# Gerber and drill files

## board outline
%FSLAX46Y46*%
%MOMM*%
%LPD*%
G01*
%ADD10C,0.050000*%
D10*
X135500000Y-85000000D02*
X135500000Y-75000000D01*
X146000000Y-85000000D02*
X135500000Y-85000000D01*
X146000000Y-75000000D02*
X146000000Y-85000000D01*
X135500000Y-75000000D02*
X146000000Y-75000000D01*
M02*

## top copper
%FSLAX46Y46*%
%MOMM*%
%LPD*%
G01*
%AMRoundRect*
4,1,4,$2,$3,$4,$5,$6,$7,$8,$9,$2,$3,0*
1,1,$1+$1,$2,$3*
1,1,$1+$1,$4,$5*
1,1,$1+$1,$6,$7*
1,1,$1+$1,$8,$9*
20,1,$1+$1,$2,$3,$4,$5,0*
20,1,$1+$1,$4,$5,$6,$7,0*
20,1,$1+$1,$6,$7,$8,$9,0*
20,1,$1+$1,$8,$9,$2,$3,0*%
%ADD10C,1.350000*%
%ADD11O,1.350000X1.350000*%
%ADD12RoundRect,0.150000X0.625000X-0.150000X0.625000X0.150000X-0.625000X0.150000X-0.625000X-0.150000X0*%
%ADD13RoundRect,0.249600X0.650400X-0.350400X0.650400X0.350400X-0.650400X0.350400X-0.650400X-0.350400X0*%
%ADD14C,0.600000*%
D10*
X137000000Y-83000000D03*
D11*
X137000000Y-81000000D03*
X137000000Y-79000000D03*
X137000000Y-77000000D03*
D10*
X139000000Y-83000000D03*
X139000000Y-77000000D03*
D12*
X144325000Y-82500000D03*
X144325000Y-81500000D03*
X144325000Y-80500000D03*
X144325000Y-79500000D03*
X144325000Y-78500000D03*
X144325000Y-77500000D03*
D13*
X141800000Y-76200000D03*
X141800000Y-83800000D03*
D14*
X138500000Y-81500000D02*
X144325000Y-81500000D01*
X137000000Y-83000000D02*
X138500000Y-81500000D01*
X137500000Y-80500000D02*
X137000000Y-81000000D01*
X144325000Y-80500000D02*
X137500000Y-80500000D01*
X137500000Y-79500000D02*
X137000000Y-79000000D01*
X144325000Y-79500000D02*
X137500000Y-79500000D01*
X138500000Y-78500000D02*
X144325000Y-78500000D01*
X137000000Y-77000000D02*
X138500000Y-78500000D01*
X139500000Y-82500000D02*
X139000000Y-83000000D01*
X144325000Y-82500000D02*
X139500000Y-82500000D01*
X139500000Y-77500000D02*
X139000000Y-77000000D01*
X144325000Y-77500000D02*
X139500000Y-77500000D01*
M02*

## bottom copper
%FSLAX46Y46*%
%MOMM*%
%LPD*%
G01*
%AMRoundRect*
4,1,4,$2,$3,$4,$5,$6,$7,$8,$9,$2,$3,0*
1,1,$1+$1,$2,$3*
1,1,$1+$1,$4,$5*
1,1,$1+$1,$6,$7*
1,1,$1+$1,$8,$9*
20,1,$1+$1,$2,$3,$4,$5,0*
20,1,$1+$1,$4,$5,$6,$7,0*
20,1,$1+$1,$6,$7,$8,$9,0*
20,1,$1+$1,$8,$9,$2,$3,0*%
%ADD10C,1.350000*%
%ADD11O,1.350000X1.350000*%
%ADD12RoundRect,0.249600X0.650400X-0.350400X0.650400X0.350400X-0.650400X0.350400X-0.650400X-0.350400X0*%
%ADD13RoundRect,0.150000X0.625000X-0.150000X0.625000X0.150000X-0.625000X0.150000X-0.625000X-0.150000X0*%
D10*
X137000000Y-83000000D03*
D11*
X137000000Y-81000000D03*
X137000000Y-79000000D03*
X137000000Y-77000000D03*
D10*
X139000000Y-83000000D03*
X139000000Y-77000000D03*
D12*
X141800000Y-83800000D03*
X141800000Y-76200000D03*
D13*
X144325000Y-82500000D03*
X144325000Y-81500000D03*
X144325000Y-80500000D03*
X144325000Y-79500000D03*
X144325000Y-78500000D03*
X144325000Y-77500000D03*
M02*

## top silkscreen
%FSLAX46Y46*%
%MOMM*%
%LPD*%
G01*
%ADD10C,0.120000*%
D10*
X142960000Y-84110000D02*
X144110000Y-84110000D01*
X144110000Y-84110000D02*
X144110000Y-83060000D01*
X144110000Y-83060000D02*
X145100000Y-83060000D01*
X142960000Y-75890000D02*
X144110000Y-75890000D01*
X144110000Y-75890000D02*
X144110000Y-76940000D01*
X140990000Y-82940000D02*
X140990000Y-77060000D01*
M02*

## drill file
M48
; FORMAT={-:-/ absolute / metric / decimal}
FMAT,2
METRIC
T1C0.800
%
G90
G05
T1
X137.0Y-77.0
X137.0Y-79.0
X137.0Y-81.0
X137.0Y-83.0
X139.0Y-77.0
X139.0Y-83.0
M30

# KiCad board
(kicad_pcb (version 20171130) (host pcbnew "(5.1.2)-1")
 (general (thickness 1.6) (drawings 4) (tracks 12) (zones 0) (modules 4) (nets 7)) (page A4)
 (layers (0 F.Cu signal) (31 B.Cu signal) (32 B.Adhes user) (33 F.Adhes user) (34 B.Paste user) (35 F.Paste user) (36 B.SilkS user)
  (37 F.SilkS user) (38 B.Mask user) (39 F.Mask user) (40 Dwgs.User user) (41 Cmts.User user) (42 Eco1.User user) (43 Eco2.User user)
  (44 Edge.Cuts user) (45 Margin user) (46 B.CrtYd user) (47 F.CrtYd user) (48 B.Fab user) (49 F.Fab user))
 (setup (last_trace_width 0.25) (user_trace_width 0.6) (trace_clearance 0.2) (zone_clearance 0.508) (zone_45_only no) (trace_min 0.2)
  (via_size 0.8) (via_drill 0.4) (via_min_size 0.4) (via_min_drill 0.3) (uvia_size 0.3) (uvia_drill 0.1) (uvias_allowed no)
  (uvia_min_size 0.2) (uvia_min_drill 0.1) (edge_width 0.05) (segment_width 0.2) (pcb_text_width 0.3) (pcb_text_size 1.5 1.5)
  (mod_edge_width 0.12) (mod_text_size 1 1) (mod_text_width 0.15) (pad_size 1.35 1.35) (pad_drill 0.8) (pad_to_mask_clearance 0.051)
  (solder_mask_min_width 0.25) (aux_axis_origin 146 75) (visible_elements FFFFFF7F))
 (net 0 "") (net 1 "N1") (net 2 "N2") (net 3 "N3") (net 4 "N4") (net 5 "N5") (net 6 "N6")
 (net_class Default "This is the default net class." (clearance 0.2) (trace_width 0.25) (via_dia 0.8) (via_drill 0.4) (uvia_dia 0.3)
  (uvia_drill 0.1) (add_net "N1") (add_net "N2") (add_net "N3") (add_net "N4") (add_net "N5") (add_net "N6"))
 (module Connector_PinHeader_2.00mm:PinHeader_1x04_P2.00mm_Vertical (layer F.Cu) (at 137 83 180)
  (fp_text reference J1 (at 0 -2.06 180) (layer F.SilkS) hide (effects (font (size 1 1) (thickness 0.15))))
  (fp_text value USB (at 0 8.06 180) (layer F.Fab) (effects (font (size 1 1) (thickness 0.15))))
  (pad 1 thru_hole circle (at 0 0 180) (size 1.35 1.35) (drill 0.8) (layers *.Cu *.Mask) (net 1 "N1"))
  (pad 2 thru_hole oval (at 0 2 180) (size 1.35 1.35) (drill 0.8) (layers *.Cu *.Mask) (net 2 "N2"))
  (pad 3 thru_hole oval (at 0 4 180) (size 1.35 1.35) (drill 0.8) (layers *.Cu *.Mask) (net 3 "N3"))
  (pad 4 thru_hole oval (at 0 6 180) (size 1.35 1.35) (drill 0.8) (layers *.Cu *.Mask) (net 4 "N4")))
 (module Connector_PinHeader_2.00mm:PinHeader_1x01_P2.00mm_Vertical (layer F.Cu) (at 139 83)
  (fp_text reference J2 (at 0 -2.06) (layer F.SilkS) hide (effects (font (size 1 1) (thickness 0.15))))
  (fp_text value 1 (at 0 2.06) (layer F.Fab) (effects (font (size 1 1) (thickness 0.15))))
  (pad 1 thru_hole circle (at 0 0) (size 1.35 1.35) (drill 0.8) (layers *.Cu *.Mask) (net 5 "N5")))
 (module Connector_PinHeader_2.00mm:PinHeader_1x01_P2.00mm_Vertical (layer F.Cu) (at 139 77)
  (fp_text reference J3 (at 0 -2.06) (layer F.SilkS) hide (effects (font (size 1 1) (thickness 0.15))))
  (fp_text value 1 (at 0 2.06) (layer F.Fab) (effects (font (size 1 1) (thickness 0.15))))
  (pad 1 thru_hole circle (at 0 0) (size 1.35 1.35) (drill 0.8) (layers *.Cu *.Mask) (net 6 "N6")))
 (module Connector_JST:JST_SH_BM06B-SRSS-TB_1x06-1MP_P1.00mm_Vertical (layer F.Cu) (at 143 80 90)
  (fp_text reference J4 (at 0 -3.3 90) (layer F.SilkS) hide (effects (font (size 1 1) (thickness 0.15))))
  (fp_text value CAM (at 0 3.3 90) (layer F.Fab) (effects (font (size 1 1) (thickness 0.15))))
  (fp_line (start -4.11 -0.04) (end -4.11 1.11) (layer F.SilkS) (width 0.12))
  (fp_line (start -4.11 1.11) (end -3.06 1.11) (layer F.SilkS) (width 0.12))
  (fp_line (start -3.06 1.11) (end -3.06 2.1) (layer F.SilkS) (width 0.12))
  (fp_line (start 4.11 -0.04) (end 4.11 1.11) (layer F.SilkS) (width 0.12))
  (fp_line (start 4.11 1.11) (end 3.06 1.11) (layer F.SilkS) (width 0.12))
  (fp_line (start -2.94 -2.01) (end 2.94 -2.01) (layer F.SilkS) (width 0.12))
  (pad 1 smd roundrect (at -2.5 1.325 90) (size 0.6 1.55) (layers F.Cu F.Paste F.Mask) (roundrect_rratio 0.25) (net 5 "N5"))
  (pad 2 smd roundrect (at -1.5 1.325 90) (size 0.6 1.55) (layers F.Cu F.Paste F.Mask) (roundrect_rratio 0.25) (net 1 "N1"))
  (pad 3 smd roundrect (at -0.5 1.325 90) (size 0.6 1.55) (layers F.Cu F.Paste F.Mask) (roundrect_rratio 0.25) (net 2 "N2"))
  (pad 4 smd roundrect (at 0.5 1.325 90) (size 0.6 1.55) (layers F.Cu F.Paste F.Mask) (roundrect_rratio 0.25) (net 3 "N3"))
  (pad 5 smd roundrect (at 1.5 1.325 90) (size 0.6 1.55) (layers F.Cu F.Paste F.Mask) (roundrect_rratio 0.25) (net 4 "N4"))
  (pad 6 smd roundrect (at 2.5 1.325 90) (size 0.6 1.55) (layers F.Cu F.Paste F.Mask) (roundrect_rratio 0.25) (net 6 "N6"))
  (pad MP smd roundrect (at -3.8 -1.2 90) (size 1.2 1.8) (layers B.Cu B.Paste B.Mask) (roundrect_rratio 0.208))
  (pad MP smd roundrect (at 3.8 -1.2 90) (size 1.2 1.8) (layers B.Cu B.Paste B.Mask) (roundrect_rratio 0.208))
  (pad 1 smd roundrect (at -2.5 1.325 90) (size 0.6 1.55) (layers B.Cu B.Paste B.Mask) (roundrect_rratio 0.25) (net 5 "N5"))
  (pad 2 smd roundrect (at -1.5 1.325 90) (size 0.6 1.55) (layers B.Cu B.Paste B.Mask) (roundrect_rratio 0.25) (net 1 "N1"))
  (pad 3 smd roundrect (at -0.5 1.325 90) (size 0.6 1.55) (layers B.Cu B.Paste B.Mask) (roundrect_rratio 0.25) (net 2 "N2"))
  (pad 4 smd roundrect (at 0.5 1.325 90) (size 0.6 1.55) (layers B.Cu B.Paste B.Mask) (roundrect_rratio 0.25) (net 3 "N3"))
  (pad 5 smd roundrect (at 1.5 1.325 90) (size 0.6 1.55) (layers B.Cu B.Paste B.Mask) (roundrect_rratio 0.25) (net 4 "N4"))
  (pad 6 smd roundrect (at 2.5 1.325 90) (size 0.6 1.55) (layers B.Cu B.Paste B.Mask) (roundrect_rratio 0.25) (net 6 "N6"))
  (pad MP smd roundrect (at 3.8 -1.2 90) (size 1.2 1.8) (layers F.Cu F.Paste F.Mask) (roundrect_rratio 0.208))
  (pad MP smd roundrect (at -3.8 -1.2 90) (size 1.2 1.8) (layers F.Cu F.Paste F.Mask) (roundrect_rratio 0.208)))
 (gr_line (start 135.5 85) (end 135.5 75) (layer Edge.Cuts) (width 0.05))
 (gr_line (start 146 85) (end 135.5 85) (layer Edge.Cuts) (width 0.05))
 (gr_line (start 146 75) (end 146 85) (layer Edge.Cuts) (width 0.05))
 (gr_line (start 135.5 75) (end 146 75) (layer Edge.Cuts) (width 0.05))
 (segment (start 138.5 81.5) (end 144.325 81.5) (width 0.6) (layer F.Cu) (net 1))
 (segment (start 137 83) (end 138.5 81.5) (width 0.6) (layer F.Cu) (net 1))
 (segment (start 137.5 80.5) (end 137 81) (width 0.6) (layer F.Cu) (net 2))
 (segment (start 144.325 80.5) (end 137.5 80.5) (width 0.6) (layer F.Cu) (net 2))
 (segment (start 137.5 79.5) (end 137 79) (width 0.6) (layer F.Cu) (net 3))
 (segment (start 144.325 79.5) (end 137.5 79.5) (width 0.6) (layer F.Cu) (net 3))
 (segment (start 138.5 78.5) (end 144.325 78.5) (width 0.6) (layer F.Cu) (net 4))
 (segment (start 137 77) (end 138.5 78.5) (width 0.6) (layer F.Cu) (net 4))
 (segment (start 139.5 82.5) (end 139 83) (width 0.6) (layer F.Cu) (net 5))
 (segment (start 144.325 82.5) (end 139.5 82.5) (width 0.6) (layer F.Cu) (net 5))
 (segment (start 139.5 77.5) (end 139 77) (width 0.6) (layer F.Cu) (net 6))
 (segment (start 144.325 77.5) (end 139.5 77.5) (width 0.6) (layer F.Cu) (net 6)))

